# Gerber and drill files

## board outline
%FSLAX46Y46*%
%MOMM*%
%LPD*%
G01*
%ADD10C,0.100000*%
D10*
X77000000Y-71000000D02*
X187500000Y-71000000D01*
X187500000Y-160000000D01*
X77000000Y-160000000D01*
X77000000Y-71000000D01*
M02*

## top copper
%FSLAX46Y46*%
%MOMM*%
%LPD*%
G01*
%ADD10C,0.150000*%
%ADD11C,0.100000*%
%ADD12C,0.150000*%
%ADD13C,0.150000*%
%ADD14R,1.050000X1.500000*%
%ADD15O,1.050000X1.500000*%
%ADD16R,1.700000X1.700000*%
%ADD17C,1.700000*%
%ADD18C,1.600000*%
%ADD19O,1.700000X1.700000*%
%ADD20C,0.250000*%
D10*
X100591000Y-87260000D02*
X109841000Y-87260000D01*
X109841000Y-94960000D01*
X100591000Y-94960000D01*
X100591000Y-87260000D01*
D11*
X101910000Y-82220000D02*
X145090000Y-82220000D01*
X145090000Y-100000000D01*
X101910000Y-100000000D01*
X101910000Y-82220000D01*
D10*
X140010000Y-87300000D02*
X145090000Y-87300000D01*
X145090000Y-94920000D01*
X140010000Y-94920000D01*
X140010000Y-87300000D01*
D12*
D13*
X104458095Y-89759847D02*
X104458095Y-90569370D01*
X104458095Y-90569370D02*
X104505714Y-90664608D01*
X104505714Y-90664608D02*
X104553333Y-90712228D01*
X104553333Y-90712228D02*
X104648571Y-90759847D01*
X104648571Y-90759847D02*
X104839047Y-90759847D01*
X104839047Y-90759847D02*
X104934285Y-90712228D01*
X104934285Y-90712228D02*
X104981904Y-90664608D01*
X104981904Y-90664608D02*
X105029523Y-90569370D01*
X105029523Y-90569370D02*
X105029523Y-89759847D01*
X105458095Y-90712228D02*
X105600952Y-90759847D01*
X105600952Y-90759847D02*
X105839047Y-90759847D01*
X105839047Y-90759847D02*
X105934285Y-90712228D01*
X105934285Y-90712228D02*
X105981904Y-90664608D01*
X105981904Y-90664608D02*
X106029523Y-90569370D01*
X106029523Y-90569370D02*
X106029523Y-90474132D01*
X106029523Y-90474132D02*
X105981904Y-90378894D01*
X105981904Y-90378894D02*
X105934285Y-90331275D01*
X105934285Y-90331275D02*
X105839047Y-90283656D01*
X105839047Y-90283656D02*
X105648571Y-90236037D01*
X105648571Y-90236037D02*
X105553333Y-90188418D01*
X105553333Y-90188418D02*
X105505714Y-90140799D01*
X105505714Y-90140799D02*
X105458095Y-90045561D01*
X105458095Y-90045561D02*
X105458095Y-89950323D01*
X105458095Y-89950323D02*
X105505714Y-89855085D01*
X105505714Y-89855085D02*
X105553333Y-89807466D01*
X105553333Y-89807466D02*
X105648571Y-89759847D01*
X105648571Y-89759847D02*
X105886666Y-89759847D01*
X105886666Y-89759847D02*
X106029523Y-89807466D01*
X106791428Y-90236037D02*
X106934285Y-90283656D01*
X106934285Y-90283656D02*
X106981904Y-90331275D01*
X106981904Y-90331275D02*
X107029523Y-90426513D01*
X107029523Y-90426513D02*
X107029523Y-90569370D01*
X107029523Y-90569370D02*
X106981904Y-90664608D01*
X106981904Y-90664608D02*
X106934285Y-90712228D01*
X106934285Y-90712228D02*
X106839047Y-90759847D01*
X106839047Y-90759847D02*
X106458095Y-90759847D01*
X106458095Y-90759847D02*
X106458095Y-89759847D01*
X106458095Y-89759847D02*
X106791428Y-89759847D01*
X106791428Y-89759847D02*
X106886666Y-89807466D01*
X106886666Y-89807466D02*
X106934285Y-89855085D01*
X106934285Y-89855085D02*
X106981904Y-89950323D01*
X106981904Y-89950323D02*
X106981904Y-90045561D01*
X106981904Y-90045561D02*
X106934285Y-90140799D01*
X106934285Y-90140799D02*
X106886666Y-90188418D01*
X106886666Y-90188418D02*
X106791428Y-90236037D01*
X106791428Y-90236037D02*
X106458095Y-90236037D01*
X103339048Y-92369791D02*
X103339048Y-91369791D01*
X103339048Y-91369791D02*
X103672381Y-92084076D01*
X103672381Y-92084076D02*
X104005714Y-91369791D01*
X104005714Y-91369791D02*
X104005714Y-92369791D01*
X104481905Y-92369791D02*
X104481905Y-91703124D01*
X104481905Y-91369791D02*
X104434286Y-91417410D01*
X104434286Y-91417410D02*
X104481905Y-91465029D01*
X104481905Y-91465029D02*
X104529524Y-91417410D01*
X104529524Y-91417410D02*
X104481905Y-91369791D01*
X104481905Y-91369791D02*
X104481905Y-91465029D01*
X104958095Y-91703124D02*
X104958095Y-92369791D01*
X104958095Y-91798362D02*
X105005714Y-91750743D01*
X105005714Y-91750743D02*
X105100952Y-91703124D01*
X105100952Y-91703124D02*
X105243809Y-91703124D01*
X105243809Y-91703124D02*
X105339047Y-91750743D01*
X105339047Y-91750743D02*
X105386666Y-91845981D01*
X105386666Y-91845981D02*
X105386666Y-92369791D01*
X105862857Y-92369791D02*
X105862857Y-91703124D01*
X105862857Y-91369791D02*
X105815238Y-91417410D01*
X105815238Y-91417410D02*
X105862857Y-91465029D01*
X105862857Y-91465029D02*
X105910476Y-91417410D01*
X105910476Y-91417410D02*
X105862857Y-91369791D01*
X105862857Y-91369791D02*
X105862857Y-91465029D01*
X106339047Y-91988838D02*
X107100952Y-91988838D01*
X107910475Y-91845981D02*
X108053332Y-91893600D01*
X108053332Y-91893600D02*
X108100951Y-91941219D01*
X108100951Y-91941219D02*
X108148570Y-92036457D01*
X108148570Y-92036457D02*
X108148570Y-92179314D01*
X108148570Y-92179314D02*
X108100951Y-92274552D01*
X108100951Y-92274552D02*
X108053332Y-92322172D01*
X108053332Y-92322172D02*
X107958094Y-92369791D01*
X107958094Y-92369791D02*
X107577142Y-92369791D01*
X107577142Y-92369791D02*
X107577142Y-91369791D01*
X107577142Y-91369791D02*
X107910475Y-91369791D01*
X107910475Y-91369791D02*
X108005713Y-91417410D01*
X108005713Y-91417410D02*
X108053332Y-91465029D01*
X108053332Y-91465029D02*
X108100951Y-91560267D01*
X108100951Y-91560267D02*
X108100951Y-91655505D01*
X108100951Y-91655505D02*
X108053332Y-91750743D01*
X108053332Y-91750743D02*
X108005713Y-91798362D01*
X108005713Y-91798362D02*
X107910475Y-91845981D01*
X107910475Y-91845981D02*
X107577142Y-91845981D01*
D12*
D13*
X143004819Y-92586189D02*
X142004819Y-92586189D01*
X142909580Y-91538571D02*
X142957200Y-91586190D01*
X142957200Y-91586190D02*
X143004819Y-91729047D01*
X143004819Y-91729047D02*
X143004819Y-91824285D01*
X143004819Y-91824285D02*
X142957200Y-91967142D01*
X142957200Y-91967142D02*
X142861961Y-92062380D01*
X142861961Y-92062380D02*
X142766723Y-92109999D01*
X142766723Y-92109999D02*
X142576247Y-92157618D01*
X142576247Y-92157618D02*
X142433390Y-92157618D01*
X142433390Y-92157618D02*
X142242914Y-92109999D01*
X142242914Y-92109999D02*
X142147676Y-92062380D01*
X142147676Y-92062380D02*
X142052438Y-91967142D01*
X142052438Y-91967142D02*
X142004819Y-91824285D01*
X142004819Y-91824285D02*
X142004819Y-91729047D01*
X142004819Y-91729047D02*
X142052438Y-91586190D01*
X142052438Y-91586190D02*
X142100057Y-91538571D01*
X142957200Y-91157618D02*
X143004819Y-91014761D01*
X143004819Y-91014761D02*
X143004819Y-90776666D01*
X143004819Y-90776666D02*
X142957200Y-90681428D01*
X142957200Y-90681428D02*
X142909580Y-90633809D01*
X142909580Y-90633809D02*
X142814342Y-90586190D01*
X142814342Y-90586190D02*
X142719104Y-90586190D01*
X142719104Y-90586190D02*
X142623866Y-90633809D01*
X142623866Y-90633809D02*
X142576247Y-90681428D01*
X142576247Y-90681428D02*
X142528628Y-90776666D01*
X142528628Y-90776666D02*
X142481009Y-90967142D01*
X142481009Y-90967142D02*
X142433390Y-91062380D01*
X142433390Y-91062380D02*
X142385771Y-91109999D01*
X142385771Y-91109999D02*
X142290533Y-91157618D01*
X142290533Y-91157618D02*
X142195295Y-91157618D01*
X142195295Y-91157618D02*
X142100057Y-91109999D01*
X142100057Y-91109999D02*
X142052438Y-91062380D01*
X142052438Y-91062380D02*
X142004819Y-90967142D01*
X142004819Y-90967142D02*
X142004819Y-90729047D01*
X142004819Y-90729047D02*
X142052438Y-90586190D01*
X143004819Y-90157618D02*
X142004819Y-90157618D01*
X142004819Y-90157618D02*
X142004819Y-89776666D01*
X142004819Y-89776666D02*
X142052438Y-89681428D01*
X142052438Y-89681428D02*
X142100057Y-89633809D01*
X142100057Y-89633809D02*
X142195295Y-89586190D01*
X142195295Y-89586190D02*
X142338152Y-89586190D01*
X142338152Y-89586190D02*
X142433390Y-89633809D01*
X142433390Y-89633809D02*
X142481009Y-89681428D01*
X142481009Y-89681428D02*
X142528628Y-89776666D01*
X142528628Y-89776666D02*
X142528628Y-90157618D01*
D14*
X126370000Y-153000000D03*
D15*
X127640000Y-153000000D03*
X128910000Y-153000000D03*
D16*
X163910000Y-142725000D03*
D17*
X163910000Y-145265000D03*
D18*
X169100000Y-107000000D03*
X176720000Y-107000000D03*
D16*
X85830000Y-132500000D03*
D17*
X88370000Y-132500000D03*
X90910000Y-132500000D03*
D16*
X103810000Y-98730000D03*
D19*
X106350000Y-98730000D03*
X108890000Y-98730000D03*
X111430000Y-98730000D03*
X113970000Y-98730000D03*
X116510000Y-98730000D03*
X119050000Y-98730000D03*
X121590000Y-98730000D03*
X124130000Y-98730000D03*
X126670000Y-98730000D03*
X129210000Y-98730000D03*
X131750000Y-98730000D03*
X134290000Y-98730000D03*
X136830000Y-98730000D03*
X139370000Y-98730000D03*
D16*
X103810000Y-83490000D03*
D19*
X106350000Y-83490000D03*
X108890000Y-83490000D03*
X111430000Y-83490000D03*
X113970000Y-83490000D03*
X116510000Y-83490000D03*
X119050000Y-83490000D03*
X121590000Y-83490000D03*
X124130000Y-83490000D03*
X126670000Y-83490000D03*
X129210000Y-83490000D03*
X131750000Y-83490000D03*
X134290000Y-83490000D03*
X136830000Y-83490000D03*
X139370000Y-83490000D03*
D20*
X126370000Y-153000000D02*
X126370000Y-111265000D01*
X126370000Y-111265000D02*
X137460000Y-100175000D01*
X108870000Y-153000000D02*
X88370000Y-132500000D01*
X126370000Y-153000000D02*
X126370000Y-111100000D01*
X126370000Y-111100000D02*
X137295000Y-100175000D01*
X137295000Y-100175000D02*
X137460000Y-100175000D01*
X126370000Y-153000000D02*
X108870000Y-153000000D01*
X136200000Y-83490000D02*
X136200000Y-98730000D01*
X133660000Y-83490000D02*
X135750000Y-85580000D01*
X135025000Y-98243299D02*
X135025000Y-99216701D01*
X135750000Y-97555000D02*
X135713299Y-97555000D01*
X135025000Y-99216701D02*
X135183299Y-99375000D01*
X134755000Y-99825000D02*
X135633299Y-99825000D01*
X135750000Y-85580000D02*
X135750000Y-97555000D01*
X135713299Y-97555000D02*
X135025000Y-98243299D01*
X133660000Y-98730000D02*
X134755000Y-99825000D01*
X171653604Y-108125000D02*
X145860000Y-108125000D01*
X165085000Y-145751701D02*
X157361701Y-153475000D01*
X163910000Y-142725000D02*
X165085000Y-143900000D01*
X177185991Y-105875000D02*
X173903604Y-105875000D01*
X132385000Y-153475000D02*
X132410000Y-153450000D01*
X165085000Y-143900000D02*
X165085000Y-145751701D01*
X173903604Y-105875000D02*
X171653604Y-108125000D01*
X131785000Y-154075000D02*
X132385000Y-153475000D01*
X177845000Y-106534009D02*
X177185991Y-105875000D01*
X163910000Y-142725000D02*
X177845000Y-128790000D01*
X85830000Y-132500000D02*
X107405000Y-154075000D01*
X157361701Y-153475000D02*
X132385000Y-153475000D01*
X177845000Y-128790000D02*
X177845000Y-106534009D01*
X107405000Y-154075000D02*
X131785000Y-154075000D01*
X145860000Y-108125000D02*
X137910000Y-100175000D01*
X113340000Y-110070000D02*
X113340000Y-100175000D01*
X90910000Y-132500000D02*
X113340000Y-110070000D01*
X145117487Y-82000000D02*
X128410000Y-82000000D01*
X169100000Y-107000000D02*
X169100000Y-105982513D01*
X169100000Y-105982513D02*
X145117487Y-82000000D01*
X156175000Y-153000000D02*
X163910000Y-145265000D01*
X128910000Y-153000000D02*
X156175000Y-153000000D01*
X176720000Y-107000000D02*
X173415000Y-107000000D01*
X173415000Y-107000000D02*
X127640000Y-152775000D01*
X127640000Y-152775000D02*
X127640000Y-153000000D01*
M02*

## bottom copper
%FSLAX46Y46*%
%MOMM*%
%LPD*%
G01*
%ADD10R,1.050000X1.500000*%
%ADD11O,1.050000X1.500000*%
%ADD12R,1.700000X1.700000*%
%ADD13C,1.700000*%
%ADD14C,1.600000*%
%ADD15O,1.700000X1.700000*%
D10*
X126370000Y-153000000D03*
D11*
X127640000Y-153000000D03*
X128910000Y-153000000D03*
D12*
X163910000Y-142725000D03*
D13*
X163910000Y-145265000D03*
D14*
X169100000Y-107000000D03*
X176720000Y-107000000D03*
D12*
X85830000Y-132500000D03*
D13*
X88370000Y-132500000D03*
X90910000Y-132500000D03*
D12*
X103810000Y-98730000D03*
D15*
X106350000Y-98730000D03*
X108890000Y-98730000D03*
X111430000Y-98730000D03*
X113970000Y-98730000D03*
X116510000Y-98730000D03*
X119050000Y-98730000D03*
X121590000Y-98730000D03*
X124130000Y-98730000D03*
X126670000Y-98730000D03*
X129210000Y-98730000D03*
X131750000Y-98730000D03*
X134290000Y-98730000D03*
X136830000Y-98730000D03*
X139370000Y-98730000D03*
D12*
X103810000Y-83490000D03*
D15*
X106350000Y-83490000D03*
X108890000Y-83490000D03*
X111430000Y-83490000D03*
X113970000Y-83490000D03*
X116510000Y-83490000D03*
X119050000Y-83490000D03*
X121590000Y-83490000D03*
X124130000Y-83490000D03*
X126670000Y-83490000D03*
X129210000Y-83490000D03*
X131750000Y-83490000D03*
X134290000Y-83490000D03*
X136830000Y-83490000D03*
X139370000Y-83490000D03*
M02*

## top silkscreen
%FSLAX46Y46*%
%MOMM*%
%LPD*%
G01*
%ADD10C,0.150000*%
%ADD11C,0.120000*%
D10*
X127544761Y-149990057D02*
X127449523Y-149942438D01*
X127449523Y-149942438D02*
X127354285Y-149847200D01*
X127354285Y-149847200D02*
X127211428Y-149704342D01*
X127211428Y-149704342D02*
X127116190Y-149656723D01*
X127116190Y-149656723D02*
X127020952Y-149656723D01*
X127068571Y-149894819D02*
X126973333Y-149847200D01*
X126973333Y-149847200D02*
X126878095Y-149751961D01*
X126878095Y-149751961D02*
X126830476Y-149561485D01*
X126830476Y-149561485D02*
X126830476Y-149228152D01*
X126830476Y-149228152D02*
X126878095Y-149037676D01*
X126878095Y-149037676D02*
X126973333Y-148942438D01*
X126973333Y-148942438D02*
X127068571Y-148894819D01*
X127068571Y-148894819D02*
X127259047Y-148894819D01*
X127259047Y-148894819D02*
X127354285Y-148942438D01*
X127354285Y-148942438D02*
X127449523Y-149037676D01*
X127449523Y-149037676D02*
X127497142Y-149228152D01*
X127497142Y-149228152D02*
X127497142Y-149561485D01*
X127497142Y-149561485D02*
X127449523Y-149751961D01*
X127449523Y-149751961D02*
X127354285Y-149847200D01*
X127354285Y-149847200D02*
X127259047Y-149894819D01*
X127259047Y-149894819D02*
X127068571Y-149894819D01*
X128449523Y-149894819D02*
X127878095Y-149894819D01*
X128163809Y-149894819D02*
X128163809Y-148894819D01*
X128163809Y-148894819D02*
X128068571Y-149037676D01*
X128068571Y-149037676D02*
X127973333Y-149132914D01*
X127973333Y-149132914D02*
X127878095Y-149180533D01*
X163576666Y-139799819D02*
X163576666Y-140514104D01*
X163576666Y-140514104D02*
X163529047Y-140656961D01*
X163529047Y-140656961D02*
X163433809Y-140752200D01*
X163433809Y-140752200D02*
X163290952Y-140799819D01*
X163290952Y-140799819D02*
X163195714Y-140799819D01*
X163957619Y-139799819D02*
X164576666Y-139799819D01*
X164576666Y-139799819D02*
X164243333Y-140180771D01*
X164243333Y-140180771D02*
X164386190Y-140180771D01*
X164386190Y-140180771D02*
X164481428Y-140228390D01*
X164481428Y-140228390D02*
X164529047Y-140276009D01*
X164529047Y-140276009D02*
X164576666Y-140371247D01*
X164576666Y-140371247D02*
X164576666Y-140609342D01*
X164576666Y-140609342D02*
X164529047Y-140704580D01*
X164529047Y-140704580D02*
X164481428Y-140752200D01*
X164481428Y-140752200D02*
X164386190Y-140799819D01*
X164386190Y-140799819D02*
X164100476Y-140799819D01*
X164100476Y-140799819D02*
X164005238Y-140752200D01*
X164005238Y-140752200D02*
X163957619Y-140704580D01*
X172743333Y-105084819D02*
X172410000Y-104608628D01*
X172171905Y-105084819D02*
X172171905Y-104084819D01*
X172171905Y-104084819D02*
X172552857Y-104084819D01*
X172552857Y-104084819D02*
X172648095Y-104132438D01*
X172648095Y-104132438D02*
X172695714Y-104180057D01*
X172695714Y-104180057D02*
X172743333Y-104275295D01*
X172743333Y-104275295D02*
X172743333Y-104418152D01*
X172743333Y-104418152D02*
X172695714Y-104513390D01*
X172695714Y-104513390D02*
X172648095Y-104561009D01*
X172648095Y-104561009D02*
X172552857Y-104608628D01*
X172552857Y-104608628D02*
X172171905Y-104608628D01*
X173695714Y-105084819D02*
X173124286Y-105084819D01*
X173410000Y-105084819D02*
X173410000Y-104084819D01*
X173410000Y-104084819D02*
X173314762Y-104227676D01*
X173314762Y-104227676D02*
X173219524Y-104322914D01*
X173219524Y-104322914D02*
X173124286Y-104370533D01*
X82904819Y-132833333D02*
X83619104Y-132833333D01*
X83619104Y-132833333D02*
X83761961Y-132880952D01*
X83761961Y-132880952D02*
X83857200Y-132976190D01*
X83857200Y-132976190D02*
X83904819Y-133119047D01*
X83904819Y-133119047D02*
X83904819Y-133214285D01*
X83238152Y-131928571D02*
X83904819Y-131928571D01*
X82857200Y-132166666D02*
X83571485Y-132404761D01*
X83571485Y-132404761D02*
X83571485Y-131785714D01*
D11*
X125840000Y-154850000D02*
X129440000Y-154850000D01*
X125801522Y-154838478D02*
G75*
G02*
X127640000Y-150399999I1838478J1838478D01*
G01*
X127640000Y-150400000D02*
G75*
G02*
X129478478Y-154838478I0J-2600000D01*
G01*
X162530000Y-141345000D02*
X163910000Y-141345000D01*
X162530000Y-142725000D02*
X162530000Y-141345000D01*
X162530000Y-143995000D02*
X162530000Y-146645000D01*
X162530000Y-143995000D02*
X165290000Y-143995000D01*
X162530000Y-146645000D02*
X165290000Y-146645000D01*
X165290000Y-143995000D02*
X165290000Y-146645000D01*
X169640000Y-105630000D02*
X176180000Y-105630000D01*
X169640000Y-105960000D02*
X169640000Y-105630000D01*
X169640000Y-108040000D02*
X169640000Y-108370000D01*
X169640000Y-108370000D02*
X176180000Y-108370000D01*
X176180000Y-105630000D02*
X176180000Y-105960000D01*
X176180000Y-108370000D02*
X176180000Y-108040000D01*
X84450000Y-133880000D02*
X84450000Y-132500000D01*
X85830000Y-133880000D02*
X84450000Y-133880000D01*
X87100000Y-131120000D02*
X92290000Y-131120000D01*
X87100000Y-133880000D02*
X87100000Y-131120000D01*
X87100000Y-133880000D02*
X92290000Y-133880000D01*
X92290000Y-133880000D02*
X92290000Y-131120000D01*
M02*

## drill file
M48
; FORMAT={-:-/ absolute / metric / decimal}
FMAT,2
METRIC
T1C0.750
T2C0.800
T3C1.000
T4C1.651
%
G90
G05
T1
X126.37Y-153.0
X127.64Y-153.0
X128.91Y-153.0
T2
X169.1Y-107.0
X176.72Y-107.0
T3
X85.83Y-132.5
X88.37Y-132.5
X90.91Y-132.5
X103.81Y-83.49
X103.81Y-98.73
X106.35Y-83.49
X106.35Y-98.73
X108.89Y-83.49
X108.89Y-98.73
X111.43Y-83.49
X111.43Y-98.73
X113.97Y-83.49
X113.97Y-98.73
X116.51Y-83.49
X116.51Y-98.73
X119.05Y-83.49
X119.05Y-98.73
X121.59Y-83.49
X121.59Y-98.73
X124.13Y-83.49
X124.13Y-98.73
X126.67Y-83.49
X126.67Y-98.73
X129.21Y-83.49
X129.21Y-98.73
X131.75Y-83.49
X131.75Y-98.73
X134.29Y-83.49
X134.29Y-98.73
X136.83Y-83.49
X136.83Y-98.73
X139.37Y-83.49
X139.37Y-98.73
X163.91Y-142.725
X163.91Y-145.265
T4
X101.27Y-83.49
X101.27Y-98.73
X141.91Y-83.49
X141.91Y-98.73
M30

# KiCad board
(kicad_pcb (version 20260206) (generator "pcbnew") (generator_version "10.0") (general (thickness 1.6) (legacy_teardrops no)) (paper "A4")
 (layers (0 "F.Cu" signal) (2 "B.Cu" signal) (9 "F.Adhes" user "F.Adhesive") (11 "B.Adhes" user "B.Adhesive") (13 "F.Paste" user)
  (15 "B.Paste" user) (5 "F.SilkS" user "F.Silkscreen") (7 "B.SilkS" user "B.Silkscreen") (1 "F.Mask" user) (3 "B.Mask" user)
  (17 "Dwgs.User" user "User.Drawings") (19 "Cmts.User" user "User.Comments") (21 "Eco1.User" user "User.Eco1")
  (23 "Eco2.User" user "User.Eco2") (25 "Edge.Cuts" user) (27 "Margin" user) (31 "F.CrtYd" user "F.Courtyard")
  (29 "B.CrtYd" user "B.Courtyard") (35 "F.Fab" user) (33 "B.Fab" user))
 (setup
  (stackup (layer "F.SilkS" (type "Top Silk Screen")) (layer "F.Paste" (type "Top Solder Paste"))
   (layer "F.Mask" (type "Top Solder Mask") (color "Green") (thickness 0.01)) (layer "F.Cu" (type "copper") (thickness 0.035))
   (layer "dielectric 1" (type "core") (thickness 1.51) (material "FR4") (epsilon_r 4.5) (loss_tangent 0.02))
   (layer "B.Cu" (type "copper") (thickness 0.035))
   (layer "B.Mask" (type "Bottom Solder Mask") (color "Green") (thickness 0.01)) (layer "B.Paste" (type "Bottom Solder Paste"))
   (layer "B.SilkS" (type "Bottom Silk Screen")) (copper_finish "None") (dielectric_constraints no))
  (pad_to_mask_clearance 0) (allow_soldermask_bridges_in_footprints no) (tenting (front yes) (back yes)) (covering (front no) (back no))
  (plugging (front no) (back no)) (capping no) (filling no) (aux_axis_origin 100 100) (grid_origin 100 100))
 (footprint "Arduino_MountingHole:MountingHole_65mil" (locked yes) (layer "F.Cu") (at 101.27 83.49)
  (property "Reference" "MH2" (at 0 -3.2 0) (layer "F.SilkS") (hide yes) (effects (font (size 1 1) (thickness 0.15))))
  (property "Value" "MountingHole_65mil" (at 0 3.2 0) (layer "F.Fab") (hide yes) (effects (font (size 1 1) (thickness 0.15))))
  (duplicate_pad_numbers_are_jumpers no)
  (pad "" np_thru_hole circle (at 0 0) (size 1.651 1.651) (drill 1.651) (layers "*.Cu" "*.Mask")))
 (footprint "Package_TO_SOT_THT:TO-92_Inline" (layer "F.Cu") (at 126.37 153)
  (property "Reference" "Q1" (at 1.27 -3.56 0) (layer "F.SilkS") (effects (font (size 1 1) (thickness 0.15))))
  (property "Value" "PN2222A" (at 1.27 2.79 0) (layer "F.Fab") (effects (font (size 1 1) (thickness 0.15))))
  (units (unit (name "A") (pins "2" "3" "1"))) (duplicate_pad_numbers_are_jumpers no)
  (fp_line (start -0.53 1.85) (end 3.07 1.85) (stroke (width 0.12) (type solid)) (layer "F.SilkS"))
  (fp_arc (start -0.568478 1.838478) (mid -1.132087 -0.994977) (end 1.27 -2.6) (stroke (width 0.12) (type solid)) (layer "F.SilkS"))
  (fp_arc (start 1.27 -2.6) (mid 3.672087 -0.994977) (end 3.108478 1.838478) (stroke (width 0.12) (type solid)) (layer "F.SilkS"))
  (pad "1" thru_hole rect (at 0 0) (size 1.05 1.5) (drill 0.75) (layers "*.Cu" "*.Mask") (remove_unused_layers no) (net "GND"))
  (pad "2" thru_hole oval (at 1.27 0) (size 1.05 1.5) (drill 0.75) (layers "*.Cu" "*.Mask") (remove_unused_layers no) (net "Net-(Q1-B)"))
  (pad "3" thru_hole oval (at 2.54 0) (size 1.05 1.5) (drill 0.75) (layers "*.Cu" "*.Mask") (remove_unused_layers no) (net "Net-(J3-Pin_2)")))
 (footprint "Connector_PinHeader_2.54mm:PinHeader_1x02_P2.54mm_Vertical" (layer "F.Cu") (at 163.91 142.725)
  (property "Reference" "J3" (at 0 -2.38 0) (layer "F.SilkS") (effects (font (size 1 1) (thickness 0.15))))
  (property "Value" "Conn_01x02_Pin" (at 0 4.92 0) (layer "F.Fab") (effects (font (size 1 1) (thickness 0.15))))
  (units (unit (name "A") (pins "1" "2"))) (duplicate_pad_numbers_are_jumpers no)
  (fp_line (start -1.38 -1.38) (end 0 -1.38) (stroke (width 0.12) (type solid)) (layer "F.SilkS"))
  (fp_line (start -1.38 0) (end -1.38 -1.38) (stroke (width 0.12) (type solid)) (layer "F.SilkS"))
  (fp_line (start -1.38 1.27) (end -1.38 3.92) (stroke (width 0.12) (type solid)) (layer "F.SilkS"))
  (fp_line (start -1.38 1.27) (end 1.38 1.27) (stroke (width 0.12) (type solid)) (layer "F.SilkS"))
  (fp_line (start -1.38 3.92) (end 1.38 3.92) (stroke (width 0.12) (type solid)) (layer "F.SilkS"))
  (fp_line (start 1.38 1.27) (end 1.38 3.92) (stroke (width 0.12) (type solid)) (layer "F.SilkS"))
  (pad "1" thru_hole rect (at 0 0) (size 1.7 1.7) (drill 1) (layers "*.Cu" "*.Mask") (remove_unused_layers no) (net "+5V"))
  (pad "2" thru_hole circle (at 0 2.54) (size 1.7 1.7) (drill 1) (layers "*.Cu" "*.Mask") (remove_unused_layers no) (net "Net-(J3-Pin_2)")))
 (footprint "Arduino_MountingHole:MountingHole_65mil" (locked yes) (layer "F.Cu") (at 141.91 98.73)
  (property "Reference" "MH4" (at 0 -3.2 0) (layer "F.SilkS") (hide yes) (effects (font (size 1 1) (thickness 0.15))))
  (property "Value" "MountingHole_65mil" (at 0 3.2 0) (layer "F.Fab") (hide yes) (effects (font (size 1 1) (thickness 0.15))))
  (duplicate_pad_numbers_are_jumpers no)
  (pad "" np_thru_hole circle (at 0 0) (size 1.651 1.651) (drill 1.651) (layers "*.Cu" "*.Mask")))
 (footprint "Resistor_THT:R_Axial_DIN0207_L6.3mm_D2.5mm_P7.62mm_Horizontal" (layer "F.Cu") (at 169.1 107)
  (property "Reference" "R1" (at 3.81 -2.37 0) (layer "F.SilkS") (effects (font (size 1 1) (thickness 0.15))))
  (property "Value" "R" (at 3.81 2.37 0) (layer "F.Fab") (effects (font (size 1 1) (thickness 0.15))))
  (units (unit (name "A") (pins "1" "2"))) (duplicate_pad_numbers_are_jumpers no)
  (fp_line (start 0.54 -1.37) (end 7.08 -1.37) (stroke (width 0.12) (type solid)) (layer "F.SilkS"))
  (fp_line (start 0.54 -1.04) (end 0.54 -1.37) (stroke (width 0.12) (type solid)) (layer "F.SilkS"))
  (fp_line (start 0.54 1.04) (end 0.54 1.37) (stroke (width 0.12) (type solid)) (layer "F.SilkS"))
  (fp_line (start 0.54 1.37) (end 7.08 1.37) (stroke (width 0.12) (type solid)) (layer "F.SilkS"))
  (fp_line (start 7.08 -1.37) (end 7.08 -1.04) (stroke (width 0.12) (type solid)) (layer "F.SilkS"))
  (fp_line (start 7.08 1.37) (end 7.08 1.04) (stroke (width 0.12) (type solid)) (layer "F.SilkS"))
  (pad "1" thru_hole circle (at 0 0) (size 1.6 1.6) (drill 0.8) (layers "*.Cu" "*.Mask") (remove_unused_layers no) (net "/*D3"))
  (pad "2" thru_hole circle (at 7.62 0) (size 1.6 1.6) (drill 0.8) (layers "*.Cu" "*.Mask") (remove_unused_layers no) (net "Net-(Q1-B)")))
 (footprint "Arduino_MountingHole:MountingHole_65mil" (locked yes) (layer "F.Cu") (at 101.27 98.73)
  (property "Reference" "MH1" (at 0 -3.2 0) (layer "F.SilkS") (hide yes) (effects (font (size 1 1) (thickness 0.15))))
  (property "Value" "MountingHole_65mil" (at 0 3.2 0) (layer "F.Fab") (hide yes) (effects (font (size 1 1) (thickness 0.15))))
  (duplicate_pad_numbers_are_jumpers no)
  (pad "" np_thru_hole circle (at 0 0) (size 1.651 1.651) (drill 1.651) (layers "*.Cu" "*.Mask")))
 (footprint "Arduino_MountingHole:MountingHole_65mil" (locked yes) (layer "F.Cu") (at 141.91 83.49)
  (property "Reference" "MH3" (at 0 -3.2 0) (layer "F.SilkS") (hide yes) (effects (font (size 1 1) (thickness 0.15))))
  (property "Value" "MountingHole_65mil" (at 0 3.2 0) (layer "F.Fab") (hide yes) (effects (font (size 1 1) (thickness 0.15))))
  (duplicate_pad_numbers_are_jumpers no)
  (pad "" np_thru_hole circle (at 0 0) (size 1.651 1.651) (drill 1.651) (layers "*.Cu" "*.Mask")))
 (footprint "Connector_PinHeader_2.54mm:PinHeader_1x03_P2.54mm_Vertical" (layer "F.Cu") (at 85.83 132.5 90)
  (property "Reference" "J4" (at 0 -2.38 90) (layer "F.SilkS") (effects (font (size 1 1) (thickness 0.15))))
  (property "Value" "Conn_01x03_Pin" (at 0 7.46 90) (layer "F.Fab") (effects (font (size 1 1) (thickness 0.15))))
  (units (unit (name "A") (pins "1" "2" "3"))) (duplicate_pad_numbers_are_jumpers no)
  (fp_line (start -1.38 -1.38) (end 0 -1.38) (stroke (width 0.12) (type solid)) (layer "F.SilkS"))
  (fp_line (start -1.38 0) (end -1.38 -1.38) (stroke (width 0.12) (type solid)) (layer "F.SilkS"))
  (fp_line (start 1.38 1.27) (end 1.38 6.46) (stroke (width 0.12) (type solid)) (layer "F.SilkS"))
  (fp_line (start -1.38 1.27) (end 1.38 1.27) (stroke (width 0.12) (type solid)) (layer "F.SilkS"))
  (fp_line (start -1.38 1.27) (end -1.38 6.46) (stroke (width 0.12) (type solid)) (layer "F.SilkS"))
  (fp_line (start -1.38 6.46) (end 1.38 6.46) (stroke (width 0.12) (type solid)) (layer "F.SilkS"))
  (pad "1" thru_hole rect (at 0 0 90) (size 1.7 1.7) (drill 1) (layers "*.Cu" "*.Mask") (remove_unused_layers no) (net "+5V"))
  (pad "2" thru_hole circle (at 0 2.54 90) (size 1.7 1.7) (drill 1) (layers "*.Cu" "*.Mask") (remove_unused_layers no) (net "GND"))
  (pad "3" thru_hole circle (at 0 5.08 90) (size 1.7 1.7) (drill 1) (layers "*.Cu" "*.Mask") (remove_unused_layers no) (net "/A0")))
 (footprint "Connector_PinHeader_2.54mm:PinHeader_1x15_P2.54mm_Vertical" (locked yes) (layer "B.Cu") (at 103.81 98.73 -90)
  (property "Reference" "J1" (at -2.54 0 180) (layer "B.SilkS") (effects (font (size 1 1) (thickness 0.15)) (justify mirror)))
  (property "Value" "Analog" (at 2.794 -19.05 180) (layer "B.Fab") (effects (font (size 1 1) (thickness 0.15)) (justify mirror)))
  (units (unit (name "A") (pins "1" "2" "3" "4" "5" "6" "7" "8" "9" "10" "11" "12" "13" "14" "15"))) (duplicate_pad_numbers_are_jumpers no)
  (pad "1" thru_hole rect (at 0 0 270) (size 1.7 1.7) (drill 1) (layers "*.Cu" "*.Mask") (remove_unused_layers no) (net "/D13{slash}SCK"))
  (pad "2" thru_hole oval (at 0 -2.54 270) (size 1.7 1.7) (drill 1) (layers "*.Cu" "*.Mask") (remove_unused_layers no) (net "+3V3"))
  (pad "3" thru_hole oval (at 0 -5.08 270) (size 1.7 1.7) (drill 1) (layers "*.Cu" "*.Mask") (remove_unused_layers no) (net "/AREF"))
  (pad "4" thru_hole oval (at 0 -7.62 270) (size 1.7 1.7) (drill 1) (layers "*.Cu" "*.Mask") (remove_unused_layers no) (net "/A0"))
  (pad "5" thru_hole oval (at 0 -10.16 270) (size 1.7 1.7) (drill 1) (layers "*.Cu" "*.Mask") (remove_unused_layers no) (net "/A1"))
  (pad "6" thru_hole oval (at 0 -12.7 270) (size 1.7 1.7) (drill 1) (layers "*.Cu" "*.Mask") (remove_unused_layers no) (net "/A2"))
  (pad "7" thru_hole oval (at 0 -15.24 270) (size 1.7 1.7) (drill 1) (layers "*.Cu" "*.Mask") (remove_unused_layers no) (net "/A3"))
  (pad "8" thru_hole oval (at 0 -17.78 270) (size 1.7 1.7) (drill 1) (layers "*.Cu" "*.Mask") (remove_unused_layers no)
   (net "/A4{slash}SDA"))
  (pad "9" thru_hole oval (at 0 -20.32 270) (size 1.7 1.7) (drill 1) (layers "*.Cu" "*.Mask") (remove_unused_layers no)
   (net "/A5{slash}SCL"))
  (pad "10" thru_hole oval (at 0 -22.86 270) (size 1.7 1.7) (drill 1) (layers "*.Cu" "*.Mask") (remove_unused_layers no) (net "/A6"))
  (pad "11" thru_hole oval (at 0 -25.4 270) (size 1.7 1.7) (drill 1) (layers "*.Cu" "*.Mask") (remove_unused_layers no) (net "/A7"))
  (pad "12" thru_hole oval (at 0 -27.94 270) (size 1.7 1.7) (drill 1) (layers "*.Cu" "*.Mask") (remove_unused_layers no) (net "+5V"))
  (pad "13" thru_hole oval (at 0 -30.48 270) (size 1.7 1.7) (drill 1) (layers "*.Cu" "*.Mask") (remove_unused_layers no) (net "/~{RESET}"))
  (pad "14" thru_hole oval (at 0 -33.02 270) (size 1.7 1.7) (drill 1) (layers "*.Cu" "*.Mask") (remove_unused_layers no) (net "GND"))
  (pad "15" thru_hole oval (at 0 -35.56 270) (size 1.7 1.7) (drill 1) (layers "*.Cu" "*.Mask") (remove_unused_layers no) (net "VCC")))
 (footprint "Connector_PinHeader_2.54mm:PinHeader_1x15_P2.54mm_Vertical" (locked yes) (layer "B.Cu") (at 103.81 83.49 -90)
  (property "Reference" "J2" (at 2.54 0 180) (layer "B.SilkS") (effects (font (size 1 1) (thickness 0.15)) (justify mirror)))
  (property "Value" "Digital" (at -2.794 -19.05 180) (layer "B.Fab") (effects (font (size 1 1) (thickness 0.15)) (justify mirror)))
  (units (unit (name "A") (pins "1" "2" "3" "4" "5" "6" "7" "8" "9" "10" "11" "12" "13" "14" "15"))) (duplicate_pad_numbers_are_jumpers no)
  (pad "1" thru_hole rect (at 0 0 270) (size 1.7 1.7) (drill 1) (layers "*.Cu" "*.Mask") (remove_unused_layers no) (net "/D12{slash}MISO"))
  (pad "2" thru_hole oval (at 0 -2.54 270) (size 1.7 1.7) (drill 1) (layers "*.Cu" "*.Mask") (remove_unused_layers no)
   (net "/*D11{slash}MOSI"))
  (pad "3" thru_hole oval (at 0 -5.08 270) (size 1.7 1.7) (drill 1) (layers "*.Cu" "*.Mask") (remove_unused_layers no)
   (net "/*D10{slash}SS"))
  (pad "4" thru_hole oval (at 0 -7.62 270) (size 1.7 1.7) (drill 1) (layers "*.Cu" "*.Mask") (remove_unused_layers no) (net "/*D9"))
  (pad "5" thru_hole oval (at 0 -10.16 270) (size 1.7 1.7) (drill 1) (layers "*.Cu" "*.Mask") (remove_unused_layers no) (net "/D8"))
  (pad "6" thru_hole oval (at 0 -12.7 270) (size 1.7 1.7) (drill 1) (layers "*.Cu" "*.Mask") (remove_unused_layers no) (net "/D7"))
  (pad "7" thru_hole oval (at 0 -15.24 270) (size 1.7 1.7) (drill 1) (layers "*.Cu" "*.Mask") (remove_unused_layers no) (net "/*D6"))
  (pad "8" thru_hole oval (at 0 -17.78 270) (size 1.7 1.7) (drill 1) (layers "*.Cu" "*.Mask") (remove_unused_layers no) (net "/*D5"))
  (pad "9" thru_hole oval (at 0 -20.32 270) (size 1.7 1.7) (drill 1) (layers "*.Cu" "*.Mask") (remove_unused_layers no) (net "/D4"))
  (pad "10" thru_hole oval (at 0 -22.86 270) (size 1.7 1.7) (drill 1) (layers "*.Cu" "*.Mask") (remove_unused_layers no) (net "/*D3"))
  (pad "11" thru_hole oval (at 0 -25.4 270) (size 1.7 1.7) (drill 1) (layers "*.Cu" "*.Mask") (remove_unused_layers no) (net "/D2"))
  (pad "12" thru_hole oval (at 0 -27.94 270) (size 1.7 1.7) (drill 1) (layers "*.Cu" "*.Mask") (remove_unused_layers no) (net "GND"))
  (pad "13" thru_hole oval (at 0 -30.48 270) (size 1.7 1.7) (drill 1) (layers "*.Cu" "*.Mask") (remove_unused_layers no) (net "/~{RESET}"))
  (pad "14" thru_hole oval (at 0 -33.02 270) (size 1.7 1.7) (drill 1) (layers "*.Cu" "*.Mask") (remove_unused_layers no)
   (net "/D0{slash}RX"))
  (pad "15" thru_hole oval (at 0 -35.56 270) (size 1.7 1.7) (drill 1) (layers "*.Cu" "*.Mask") (remove_unused_layers no)
   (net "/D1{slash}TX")))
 (gr_rect (start 100.591 87.26) (end 109.841 94.96) (stroke (width 0.15) (type solid)) (fill no) (layer "F.Cu") (net "/*D3"))
 (gr_rect (start 101.91 82.22) (end 145.09 100) (stroke (width 0.1) (type solid)) (fill no) (layer "F.Cu") (net "/*D3"))
 (gr_rect (start 140.01 87.3) (end 145.09 94.92) (stroke (width 0.15) (type solid)) (fill no) (layer "F.Cu") (net "/*D3"))
 (gr_rect (start 77 71) (end 187.5 160) (stroke (width 0.1) (type default)) (fill no) (layer "Edge.Cuts"))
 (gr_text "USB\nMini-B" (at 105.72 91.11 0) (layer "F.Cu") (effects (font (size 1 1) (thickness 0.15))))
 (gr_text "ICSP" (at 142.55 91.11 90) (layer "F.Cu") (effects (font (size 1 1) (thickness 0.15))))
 (segment (start 126.37 153) (end 126.37 111.265) (width 0.25) (layer "F.Cu") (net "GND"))
 (segment (start 126.37 111.265) (end 137.46 100.175) (width 0.25) (layer "F.Cu") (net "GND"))
 (segment (start 108.87 153) (end 88.37 132.5) (width 0.25) (layer "F.Cu") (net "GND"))
 (segment (start 126.37 153) (end 126.37 111.1) (width 0.25) (layer "F.Cu") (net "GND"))
 (segment (start 126.37 111.1) (end 137.295 100.175) (width 0.25) (layer "F.Cu") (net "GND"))
 (segment (start 137.295 100.175) (end 137.46 100.175) (width 0.25) (layer "F.Cu") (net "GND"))
 (segment (start 126.37 153) (end 108.87 153) (width 0.25) (layer "F.Cu") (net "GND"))
 (segment (start 136.2 83.49) (end 136.2 98.73) (width 0.25) (layer "F.Cu") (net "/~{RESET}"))
 (segment (start 133.66 83.49) (end 135.75 85.58) (width 0.25) (layer "F.Cu") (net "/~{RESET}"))
 (segment (start 135.025 98.243299) (end 135.025 99.216701) (width 0.25) (layer "F.Cu") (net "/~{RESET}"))
 (segment (start 135.75 97.555) (end 135.713299 97.555) (width 0.25) (layer "F.Cu") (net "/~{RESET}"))
 (segment (start 135.025 99.216701) (end 135.183299 99.375) (width 0.25) (layer "F.Cu") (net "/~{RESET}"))
 (segment (start 134.755 99.825) (end 135.633299 99.825) (width 0.25) (layer "F.Cu") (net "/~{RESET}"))
 (segment (start 135.75 85.58) (end 135.75 97.555) (width 0.25) (layer "F.Cu") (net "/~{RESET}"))
 (segment (start 135.713299 97.555) (end 135.025 98.243299) (width 0.25) (layer "F.Cu") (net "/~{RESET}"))
 (segment (start 133.66 98.73) (end 134.755 99.825) (width 0.25) (layer "F.Cu") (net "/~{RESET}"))
 (segment (start 171.653604 108.125) (end 145.86 108.125) (width 0.25) (layer "F.Cu") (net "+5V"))
 (segment (start 165.085 145.751701) (end 157.361701 153.475) (width 0.25) (layer "F.Cu") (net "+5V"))
 (segment (start 163.91 142.725) (end 165.085 143.9) (width 0.25) (layer "F.Cu") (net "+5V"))
 (segment (start 177.185991 105.875) (end 173.903604 105.875) (width 0.25) (layer "F.Cu") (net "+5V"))
 (segment (start 132.385 153.475) (end 132.41 153.45) (width 0.25) (layer "F.Cu") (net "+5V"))
 (segment (start 165.085 143.9) (end 165.085 145.751701) (width 0.25) (layer "F.Cu") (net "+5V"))
 (segment (start 173.903604 105.875) (end 171.653604 108.125) (width 0.25) (layer "F.Cu") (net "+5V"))
 (segment (start 131.785 154.075) (end 132.385 153.475) (width 0.25) (layer "F.Cu") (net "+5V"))
 (segment (start 177.845 106.534009) (end 177.185991 105.875) (width 0.25) (layer "F.Cu") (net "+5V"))
 (segment (start 163.91 142.725) (end 177.845 128.79) (width 0.25) (layer "F.Cu") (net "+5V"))
 (segment (start 85.83 132.5) (end 107.405 154.075) (width 0.25) (layer "F.Cu") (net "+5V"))
 (segment (start 157.361701 153.475) (end 132.385 153.475) (width 0.25) (layer "F.Cu") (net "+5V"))
 (segment (start 177.845 128.79) (end 177.845 106.534009) (width 0.25) (layer "F.Cu") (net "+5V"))
 (segment (start 107.405 154.075) (end 131.785 154.075) (width 0.25) (layer "F.Cu") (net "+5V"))
 (segment (start 145.86 108.125) (end 137.91 100.175) (width 0.25) (layer "F.Cu") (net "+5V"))
 (segment (start 113.34 110.07) (end 113.34 100.175) (width 0.25) (layer "F.Cu") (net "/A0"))
 (segment (start 90.91 132.5) (end 113.34 110.07) (width 0.25) (layer "F.Cu") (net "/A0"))
 (segment (start 145.117487 82) (end 128.41 82) (width 0.25) (layer "F.Cu") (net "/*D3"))
 (segment (start 169.1 107) (end 169.1 105.982513) (width 0.25) (layer "F.Cu") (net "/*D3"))
 (segment (start 169.1 105.982513) (end 145.117487 82) (width 0.25) (layer "F.Cu") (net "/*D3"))
 (segment (start 156.175 153) (end 163.91 145.265) (width 0.25) (layer "F.Cu") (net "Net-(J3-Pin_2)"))
 (segment (start 128.91 153) (end 156.175 153) (width 0.25) (layer "F.Cu") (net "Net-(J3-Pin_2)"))
 (segment (start 176.72 107) (end 173.415 107) (width 0.25) (layer "F.Cu") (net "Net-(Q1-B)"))
 (segment (start 173.415 107) (end 127.64 152.775) (width 0.25) (layer "F.Cu") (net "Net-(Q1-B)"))
 (segment (start 127.64 152.775) (end 127.64 153) (width 0.25) (layer "F.Cu") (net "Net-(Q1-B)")))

